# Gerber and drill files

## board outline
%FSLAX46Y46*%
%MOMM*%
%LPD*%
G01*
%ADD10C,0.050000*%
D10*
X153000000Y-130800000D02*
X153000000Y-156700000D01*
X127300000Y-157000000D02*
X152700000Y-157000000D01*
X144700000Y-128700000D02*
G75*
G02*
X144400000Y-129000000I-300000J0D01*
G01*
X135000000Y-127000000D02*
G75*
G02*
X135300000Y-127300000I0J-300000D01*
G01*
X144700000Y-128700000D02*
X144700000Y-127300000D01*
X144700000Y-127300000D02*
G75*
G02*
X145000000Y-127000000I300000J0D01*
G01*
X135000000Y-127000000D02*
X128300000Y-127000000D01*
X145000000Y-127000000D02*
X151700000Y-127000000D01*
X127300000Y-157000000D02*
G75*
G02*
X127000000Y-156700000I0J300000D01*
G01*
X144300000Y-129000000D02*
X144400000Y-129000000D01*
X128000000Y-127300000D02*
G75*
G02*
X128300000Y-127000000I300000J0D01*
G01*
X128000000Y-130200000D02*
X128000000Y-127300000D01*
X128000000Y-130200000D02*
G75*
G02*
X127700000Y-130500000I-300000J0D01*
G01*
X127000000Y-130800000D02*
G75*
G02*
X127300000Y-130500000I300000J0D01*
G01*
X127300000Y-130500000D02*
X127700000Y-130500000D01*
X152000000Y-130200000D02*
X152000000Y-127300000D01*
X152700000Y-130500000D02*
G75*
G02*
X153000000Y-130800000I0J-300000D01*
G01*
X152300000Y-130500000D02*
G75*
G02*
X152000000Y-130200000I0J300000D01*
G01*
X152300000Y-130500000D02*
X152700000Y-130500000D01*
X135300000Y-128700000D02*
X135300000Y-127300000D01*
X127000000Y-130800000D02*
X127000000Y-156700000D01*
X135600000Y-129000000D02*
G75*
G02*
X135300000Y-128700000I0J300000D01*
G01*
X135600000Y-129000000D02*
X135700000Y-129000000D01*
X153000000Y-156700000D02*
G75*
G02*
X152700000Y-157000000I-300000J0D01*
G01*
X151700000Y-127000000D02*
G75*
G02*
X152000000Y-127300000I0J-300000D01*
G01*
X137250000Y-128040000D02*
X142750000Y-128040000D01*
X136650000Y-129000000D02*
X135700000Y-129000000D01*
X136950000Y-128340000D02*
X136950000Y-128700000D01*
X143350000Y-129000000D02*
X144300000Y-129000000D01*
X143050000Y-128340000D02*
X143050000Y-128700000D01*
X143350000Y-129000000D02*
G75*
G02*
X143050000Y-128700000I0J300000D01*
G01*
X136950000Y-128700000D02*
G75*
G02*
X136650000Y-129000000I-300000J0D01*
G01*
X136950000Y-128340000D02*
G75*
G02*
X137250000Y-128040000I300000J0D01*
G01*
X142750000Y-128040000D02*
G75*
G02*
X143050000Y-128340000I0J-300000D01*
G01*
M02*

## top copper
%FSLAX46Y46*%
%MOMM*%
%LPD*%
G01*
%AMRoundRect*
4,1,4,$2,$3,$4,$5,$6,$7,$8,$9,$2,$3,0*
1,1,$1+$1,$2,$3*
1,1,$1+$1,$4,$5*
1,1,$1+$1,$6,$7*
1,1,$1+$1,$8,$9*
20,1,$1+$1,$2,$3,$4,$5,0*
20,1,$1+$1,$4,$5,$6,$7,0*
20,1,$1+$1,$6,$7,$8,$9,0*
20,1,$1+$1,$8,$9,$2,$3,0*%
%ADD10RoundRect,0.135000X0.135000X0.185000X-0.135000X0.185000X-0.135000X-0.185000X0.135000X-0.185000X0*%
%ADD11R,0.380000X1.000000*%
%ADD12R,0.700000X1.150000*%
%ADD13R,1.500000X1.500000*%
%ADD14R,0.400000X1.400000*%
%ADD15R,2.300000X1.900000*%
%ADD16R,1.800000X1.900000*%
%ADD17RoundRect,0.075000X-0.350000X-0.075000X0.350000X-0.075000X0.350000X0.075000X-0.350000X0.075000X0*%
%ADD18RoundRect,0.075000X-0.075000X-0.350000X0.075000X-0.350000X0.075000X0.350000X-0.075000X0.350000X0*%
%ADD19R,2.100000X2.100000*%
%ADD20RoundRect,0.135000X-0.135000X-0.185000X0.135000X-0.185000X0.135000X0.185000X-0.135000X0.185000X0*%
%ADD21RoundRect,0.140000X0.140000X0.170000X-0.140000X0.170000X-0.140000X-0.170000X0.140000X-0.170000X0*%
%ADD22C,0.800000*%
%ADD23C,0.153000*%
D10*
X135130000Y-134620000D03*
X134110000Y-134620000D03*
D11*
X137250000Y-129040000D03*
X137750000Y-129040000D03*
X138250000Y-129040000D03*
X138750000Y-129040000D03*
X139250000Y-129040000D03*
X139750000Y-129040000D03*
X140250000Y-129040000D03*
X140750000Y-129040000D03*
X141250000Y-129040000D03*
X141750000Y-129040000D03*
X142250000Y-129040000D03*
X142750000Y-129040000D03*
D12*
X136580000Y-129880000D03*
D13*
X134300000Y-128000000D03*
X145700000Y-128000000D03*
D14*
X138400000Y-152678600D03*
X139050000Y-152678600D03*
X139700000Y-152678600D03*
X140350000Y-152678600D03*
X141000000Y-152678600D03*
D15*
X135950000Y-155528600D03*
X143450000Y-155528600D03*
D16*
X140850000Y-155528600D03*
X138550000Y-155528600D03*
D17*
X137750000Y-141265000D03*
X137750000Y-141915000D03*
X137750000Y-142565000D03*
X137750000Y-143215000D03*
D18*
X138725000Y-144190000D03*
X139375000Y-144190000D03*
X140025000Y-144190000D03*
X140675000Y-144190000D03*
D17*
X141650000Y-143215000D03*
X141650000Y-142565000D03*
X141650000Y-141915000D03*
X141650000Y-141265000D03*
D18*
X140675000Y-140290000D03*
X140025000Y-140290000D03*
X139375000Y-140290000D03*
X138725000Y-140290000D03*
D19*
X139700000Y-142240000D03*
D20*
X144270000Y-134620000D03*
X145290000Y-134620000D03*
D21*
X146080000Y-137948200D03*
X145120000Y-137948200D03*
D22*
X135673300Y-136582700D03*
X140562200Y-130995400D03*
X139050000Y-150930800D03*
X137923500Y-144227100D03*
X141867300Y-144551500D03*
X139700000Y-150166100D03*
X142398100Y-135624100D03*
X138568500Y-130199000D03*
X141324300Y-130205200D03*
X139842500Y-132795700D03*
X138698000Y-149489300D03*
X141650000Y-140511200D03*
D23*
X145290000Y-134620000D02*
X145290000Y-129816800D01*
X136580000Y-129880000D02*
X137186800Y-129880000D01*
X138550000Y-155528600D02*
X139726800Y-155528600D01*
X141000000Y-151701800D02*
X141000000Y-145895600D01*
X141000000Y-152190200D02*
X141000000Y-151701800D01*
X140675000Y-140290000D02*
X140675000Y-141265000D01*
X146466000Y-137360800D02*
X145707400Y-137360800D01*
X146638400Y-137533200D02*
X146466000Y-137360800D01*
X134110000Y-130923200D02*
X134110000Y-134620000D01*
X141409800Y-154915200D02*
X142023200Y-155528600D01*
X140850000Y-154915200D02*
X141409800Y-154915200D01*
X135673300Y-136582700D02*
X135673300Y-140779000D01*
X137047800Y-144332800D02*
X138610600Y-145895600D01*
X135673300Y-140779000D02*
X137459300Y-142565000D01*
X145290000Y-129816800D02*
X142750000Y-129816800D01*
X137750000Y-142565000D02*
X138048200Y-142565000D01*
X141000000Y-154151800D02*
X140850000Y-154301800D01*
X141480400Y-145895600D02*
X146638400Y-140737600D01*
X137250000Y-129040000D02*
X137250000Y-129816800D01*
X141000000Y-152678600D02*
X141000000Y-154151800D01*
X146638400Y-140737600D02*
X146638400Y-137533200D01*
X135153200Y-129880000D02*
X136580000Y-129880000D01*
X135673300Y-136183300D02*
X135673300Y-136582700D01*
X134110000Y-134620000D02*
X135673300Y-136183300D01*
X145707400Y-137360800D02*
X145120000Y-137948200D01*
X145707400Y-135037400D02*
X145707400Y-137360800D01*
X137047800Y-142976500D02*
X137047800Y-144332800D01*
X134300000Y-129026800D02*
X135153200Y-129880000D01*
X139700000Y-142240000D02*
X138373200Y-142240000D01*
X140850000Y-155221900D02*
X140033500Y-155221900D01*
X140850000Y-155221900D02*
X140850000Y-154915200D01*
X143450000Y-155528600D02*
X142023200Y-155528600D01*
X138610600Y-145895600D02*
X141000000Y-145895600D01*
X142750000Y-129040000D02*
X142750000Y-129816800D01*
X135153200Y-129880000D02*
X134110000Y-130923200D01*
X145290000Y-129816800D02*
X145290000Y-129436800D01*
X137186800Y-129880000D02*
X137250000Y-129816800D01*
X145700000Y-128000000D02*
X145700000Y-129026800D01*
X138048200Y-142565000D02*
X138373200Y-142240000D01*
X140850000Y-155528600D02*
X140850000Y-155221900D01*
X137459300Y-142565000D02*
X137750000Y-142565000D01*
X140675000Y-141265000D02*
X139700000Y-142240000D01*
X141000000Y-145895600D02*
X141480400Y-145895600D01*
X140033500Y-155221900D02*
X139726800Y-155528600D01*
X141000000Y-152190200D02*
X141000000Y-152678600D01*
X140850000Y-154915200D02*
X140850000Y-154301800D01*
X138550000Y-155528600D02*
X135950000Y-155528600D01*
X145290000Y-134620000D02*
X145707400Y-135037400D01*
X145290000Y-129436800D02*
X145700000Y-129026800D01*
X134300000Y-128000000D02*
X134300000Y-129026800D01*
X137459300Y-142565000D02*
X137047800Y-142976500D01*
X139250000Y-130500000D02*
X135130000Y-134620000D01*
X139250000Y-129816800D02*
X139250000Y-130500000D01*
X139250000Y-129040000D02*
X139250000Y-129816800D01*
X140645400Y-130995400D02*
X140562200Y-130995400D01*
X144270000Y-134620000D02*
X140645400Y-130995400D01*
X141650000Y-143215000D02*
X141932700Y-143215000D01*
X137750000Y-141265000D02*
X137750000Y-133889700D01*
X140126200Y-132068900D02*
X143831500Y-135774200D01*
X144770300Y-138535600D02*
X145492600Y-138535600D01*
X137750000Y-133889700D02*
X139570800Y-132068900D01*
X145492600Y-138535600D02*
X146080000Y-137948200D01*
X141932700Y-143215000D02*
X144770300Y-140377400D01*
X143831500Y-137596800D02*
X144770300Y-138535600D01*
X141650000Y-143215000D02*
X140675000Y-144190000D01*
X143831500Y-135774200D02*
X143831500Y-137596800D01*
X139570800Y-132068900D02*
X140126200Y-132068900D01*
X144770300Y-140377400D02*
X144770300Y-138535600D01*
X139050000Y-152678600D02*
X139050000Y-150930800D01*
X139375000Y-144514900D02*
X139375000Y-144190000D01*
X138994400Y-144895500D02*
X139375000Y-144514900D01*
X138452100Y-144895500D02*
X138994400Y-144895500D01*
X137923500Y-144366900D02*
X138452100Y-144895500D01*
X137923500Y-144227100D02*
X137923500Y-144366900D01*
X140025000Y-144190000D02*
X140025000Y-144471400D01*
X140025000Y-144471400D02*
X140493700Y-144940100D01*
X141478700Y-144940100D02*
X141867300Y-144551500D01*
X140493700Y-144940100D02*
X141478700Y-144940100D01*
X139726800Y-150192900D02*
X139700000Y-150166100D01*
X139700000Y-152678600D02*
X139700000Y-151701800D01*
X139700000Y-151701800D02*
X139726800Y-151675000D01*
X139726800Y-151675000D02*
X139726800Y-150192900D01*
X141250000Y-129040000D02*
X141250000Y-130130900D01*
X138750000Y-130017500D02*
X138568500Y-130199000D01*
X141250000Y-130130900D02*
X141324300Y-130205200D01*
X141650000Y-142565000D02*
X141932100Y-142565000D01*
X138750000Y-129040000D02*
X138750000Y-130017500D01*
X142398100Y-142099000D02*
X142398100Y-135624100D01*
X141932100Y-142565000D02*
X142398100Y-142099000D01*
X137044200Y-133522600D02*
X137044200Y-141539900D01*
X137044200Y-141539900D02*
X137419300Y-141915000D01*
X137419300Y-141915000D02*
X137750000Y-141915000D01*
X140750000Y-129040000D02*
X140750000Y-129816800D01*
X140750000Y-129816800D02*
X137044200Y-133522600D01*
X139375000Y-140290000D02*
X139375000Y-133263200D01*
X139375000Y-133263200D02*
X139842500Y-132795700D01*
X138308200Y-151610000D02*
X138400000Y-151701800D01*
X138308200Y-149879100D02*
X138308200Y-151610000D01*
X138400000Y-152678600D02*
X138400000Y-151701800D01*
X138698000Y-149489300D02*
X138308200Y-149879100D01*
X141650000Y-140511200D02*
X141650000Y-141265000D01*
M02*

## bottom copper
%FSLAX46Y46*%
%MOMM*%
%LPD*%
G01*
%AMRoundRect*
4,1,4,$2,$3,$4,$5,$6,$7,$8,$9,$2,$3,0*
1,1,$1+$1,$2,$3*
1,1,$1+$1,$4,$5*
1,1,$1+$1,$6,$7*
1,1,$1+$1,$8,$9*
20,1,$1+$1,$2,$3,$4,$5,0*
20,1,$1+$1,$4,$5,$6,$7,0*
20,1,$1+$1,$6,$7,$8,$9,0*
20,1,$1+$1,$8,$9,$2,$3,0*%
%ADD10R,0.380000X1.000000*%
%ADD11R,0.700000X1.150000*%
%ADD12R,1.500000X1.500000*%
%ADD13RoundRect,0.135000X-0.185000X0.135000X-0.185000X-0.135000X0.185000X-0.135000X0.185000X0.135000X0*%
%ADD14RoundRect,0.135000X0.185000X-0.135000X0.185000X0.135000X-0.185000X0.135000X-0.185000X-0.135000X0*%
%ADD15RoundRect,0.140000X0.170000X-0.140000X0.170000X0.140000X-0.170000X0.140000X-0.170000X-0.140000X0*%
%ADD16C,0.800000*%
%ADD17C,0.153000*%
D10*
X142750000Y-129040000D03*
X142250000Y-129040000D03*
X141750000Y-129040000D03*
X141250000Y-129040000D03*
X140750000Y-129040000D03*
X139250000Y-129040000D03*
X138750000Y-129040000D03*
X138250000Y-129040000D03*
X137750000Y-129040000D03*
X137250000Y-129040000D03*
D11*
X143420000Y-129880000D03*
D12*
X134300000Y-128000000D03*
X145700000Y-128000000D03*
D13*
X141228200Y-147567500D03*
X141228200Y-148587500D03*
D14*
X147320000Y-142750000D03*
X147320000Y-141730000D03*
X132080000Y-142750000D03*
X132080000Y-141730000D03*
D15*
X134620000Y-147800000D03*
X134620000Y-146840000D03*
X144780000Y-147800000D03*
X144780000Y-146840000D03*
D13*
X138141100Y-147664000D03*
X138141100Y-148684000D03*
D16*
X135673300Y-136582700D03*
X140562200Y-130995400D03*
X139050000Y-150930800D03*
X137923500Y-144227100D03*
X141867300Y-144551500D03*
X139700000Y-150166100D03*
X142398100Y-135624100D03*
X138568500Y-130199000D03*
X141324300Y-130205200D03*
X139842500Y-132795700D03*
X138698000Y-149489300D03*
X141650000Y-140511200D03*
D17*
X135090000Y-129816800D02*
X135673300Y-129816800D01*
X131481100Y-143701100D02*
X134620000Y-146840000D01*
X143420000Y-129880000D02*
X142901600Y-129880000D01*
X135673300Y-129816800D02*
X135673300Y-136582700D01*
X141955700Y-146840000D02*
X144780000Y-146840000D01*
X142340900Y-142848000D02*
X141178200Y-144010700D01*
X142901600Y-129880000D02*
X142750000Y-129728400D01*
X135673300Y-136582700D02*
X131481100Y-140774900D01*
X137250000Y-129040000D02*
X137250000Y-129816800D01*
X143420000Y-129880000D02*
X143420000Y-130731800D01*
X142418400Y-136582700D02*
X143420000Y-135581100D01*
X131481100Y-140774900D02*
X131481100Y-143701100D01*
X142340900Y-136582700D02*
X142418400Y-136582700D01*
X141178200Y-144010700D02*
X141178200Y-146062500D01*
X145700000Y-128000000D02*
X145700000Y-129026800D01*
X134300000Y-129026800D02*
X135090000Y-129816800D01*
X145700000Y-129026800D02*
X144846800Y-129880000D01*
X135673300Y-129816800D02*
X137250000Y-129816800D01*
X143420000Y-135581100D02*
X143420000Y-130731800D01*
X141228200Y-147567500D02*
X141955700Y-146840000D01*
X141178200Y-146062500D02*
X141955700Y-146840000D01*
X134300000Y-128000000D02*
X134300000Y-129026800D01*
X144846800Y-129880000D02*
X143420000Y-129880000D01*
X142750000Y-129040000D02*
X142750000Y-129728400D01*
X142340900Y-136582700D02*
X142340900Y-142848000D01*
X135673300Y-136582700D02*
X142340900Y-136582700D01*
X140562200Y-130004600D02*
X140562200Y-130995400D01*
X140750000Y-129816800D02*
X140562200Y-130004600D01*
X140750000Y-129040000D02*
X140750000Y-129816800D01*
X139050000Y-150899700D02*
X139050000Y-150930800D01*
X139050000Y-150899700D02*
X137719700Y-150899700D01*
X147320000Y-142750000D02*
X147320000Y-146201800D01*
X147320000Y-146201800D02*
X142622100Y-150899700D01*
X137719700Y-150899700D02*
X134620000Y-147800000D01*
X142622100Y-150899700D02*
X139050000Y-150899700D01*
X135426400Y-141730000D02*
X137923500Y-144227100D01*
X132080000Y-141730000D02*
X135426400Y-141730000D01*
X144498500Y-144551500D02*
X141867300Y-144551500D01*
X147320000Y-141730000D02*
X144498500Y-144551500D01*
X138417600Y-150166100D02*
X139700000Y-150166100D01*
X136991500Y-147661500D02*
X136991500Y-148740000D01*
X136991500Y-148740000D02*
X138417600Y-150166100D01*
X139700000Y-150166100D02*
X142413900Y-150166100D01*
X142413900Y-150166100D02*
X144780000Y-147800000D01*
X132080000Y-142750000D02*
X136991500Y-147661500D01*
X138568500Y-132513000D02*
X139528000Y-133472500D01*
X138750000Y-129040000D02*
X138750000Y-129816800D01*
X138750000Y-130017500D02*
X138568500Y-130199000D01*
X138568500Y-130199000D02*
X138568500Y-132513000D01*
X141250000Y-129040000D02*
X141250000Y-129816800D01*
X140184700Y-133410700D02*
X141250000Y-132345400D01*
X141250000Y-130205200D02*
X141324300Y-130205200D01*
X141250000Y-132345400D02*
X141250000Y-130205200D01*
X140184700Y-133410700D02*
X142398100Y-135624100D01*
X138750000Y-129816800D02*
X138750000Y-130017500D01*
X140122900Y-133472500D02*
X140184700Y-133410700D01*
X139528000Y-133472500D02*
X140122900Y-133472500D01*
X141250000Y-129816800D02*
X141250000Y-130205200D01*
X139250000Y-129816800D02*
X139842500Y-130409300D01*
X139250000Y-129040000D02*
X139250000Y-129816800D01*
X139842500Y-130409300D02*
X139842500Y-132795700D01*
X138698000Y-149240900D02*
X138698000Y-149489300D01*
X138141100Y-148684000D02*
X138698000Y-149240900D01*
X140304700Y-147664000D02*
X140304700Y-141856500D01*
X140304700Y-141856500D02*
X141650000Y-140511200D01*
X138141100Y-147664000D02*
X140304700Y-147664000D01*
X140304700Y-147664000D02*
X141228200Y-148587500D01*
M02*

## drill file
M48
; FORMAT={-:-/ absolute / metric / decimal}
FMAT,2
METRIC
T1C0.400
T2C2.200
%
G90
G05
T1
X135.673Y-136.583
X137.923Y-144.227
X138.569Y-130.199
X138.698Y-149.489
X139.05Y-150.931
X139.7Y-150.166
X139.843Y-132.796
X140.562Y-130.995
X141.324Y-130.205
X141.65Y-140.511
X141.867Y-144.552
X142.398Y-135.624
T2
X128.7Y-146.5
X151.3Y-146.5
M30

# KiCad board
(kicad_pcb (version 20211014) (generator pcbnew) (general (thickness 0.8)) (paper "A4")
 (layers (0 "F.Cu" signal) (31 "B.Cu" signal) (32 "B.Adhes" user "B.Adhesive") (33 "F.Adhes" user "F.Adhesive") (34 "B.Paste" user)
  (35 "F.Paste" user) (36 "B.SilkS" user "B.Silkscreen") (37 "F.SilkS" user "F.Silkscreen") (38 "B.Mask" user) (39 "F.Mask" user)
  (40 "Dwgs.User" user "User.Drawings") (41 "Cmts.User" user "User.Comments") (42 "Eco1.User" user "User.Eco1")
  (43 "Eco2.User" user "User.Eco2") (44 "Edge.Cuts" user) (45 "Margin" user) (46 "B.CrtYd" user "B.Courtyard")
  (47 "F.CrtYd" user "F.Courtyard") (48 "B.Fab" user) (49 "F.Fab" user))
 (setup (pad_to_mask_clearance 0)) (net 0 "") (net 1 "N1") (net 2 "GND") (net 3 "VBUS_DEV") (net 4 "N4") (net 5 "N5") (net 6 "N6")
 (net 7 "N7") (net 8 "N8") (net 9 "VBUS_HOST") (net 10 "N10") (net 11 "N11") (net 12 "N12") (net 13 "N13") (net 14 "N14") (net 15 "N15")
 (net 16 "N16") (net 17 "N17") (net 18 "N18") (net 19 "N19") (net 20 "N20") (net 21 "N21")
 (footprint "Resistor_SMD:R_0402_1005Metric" (layer "F.Cu") (at 134.62 134.62 180)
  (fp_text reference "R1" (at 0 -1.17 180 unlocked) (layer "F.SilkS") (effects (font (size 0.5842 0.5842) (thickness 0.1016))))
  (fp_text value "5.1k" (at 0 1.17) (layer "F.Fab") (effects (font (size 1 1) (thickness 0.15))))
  (pad "1" smd roundrect (at -0.51 0 180) (size 0.54 0.64) (layers "F.Cu" "F.Paste" "F.Mask") (roundrect_rratio 0.25) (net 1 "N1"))
  (pad "2" smd roundrect (at 0.51 0 180) (size 0.54 0.64) (layers "F.Cu" "F.Paste" "F.Mask") (roundrect_rratio 0.25) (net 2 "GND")))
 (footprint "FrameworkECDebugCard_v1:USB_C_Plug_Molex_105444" (layer "F.Cu") (at 140 129)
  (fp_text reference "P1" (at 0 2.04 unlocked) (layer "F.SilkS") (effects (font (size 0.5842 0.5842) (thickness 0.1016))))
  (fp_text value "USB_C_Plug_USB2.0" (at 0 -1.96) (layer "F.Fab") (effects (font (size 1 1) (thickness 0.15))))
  (fp_line (start -2.75 -0.96) (end 2.75 -0.96) (layer "Edge.Cuts") (width 0.05))
  (fp_line (start -3.35 0) (end -4.3 0) (layer "Edge.Cuts") (width 0.05))
  (fp_line (start -3.05 -0.66) (end -3.05 -0.3) (layer "Edge.Cuts") (width 0.05))
  (fp_line (start 3.35 0) (end 4.3 0) (layer "Edge.Cuts") (width 0.05))
  (fp_line (start 3.05 -0.66) (end 3.05 -0.3) (layer "Edge.Cuts") (width 0.05))
  (fp_arc (start 3.35 0) (mid 3.137868 -0.087868) (end 3.05 -0.3) (layer "Edge.Cuts") (width 0.05))
  (fp_arc (start -3.05 -0.3) (mid -3.137868 -0.087868) (end -3.35 0) (layer "Edge.Cuts") (width 0.05))
  (fp_arc (start -3.05 -0.66) (mid -2.962132 -0.872132) (end -2.75 -0.96) (layer "Edge.Cuts") (width 0.05))
  (fp_arc (start 2.75 -0.96) (mid 2.962132 -0.872132) (end 3.05 -0.66) (layer "Edge.Cuts") (width 0.05))
  (pad "A1" smd rect locked (at -2.75 0.04) (size 0.38 1) (layers "F.Cu" "F.Paste" "F.Mask") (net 2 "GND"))
  (pad "A2" smd rect locked (at -2.25 0.04) (size 0.38 1) (layers "F.Cu" "F.Paste" "F.Mask"))
  (pad "A3" smd rect locked (at -1.75 0.04) (size 0.38 1) (layers "F.Cu" "F.Paste" "F.Mask"))
  (pad "A4" smd rect locked (at -1.25 0.04) (size 0.38 1) (layers "F.Cu" "F.Paste" "F.Mask") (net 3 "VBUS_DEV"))
  (pad "A5" smd rect locked (at -0.75 0.04) (size 0.38 1) (layers "F.Cu" "F.Paste" "F.Mask") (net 1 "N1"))
  (pad "A6" smd rect locked (at -0.25 0.04) (size 0.38 1) (layers "F.Cu" "F.Paste" "F.Mask") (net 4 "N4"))
  (pad "A7" smd rect locked (at 0.25 0.04) (size 0.38 1) (layers "F.Cu" "F.Paste" "F.Mask") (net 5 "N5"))
  (pad "A8" smd rect locked (at 0.75 0.04) (size 0.38 1) (layers "F.Cu" "F.Paste" "F.Mask") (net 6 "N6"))
  (pad "A9" smd rect locked (at 1.25 0.04) (size 0.38 1) (layers "F.Cu" "F.Paste" "F.Mask") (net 3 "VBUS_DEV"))
  (pad "A10" smd rect locked (at 1.75 0.04) (size 0.38 1) (layers "F.Cu" "F.Paste" "F.Mask"))
  (pad "A11" smd rect locked (at 2.25 0.04) (size 0.38 1) (layers "F.Cu" "F.Paste" "F.Mask"))
  (pad "A12" smd rect locked (at 2.75 0.04) (size 0.38 1) (layers "F.Cu" "F.Paste" "F.Mask") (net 2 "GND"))
  (pad "B1" smd rect locked (at 2.75 0.04) (size 0.38 1) (layers "B.Cu" "B.Paste" "B.Mask") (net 2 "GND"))
  (pad "B2" smd rect locked (at 2.25 0.04) (size 0.38 1) (layers "B.Cu" "B.Paste" "B.Mask"))
  (pad "B3" smd rect locked (at 1.75 0.04) (size 0.38 1) (layers "B.Cu" "B.Paste" "B.Mask"))
  (pad "B4" smd rect locked (at 1.25 0.04) (size 0.38 1) (layers "B.Cu" "B.Paste" "B.Mask") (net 3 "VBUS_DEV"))
  (pad "B5" smd rect locked (at 0.75 0.04) (size 0.38 1) (layers "B.Cu" "B.Paste" "B.Mask") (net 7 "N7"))
  (pad "B8" smd rect locked (at -0.75 0.04) (size 0.38 1) (layers "B.Cu" "B.Paste" "B.Mask") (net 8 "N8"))
  (pad "B9" smd rect locked (at -1.25 0.04) (size 0.38 1) (layers "B.Cu" "B.Paste" "B.Mask") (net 3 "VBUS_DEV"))
  (pad "B10" smd rect locked (at -1.75 0.04) (size 0.38 1) (layers "B.Cu" "B.Paste" "B.Mask"))
  (pad "B11" smd rect locked (at -2.25 0.04) (size 0.38 1) (layers "B.Cu" "B.Paste" "B.Mask"))
  (pad "B12" smd rect locked (at -2.75 0.04) (size 0.38 1) (layers "B.Cu" "B.Paste" "B.Mask") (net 2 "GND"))
  (pad "S1" smd rect locked (at 3.42 0.88) (size 0.7 1.15) (layers "B.Cu" "B.Paste" "B.Mask") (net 2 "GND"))
  (pad "S1" smd rect locked (at -3.42 0.88) (size 0.7 1.15) (layers "F.Cu" "F.Paste" "F.Mask") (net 2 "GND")))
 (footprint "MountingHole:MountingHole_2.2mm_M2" (layer "F.Cu") (at 128.7 146.5)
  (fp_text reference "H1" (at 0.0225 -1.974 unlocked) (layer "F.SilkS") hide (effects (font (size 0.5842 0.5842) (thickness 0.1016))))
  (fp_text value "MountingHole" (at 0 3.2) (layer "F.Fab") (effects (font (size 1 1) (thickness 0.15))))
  (pad "" np_thru_hole circle locked (at 0 0) (size 2.2 2.2) (drill 2.2) (layers *.Cu *.Mask)))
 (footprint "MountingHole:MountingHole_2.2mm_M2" (layer "F.Cu") (at 151.3 146.5)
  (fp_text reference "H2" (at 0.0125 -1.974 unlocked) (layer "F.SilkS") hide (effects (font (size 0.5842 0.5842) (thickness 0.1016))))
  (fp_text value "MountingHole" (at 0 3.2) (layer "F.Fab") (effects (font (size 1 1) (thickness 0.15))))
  (pad "" np_thru_hole circle locked (at 0 0) (size 2.2 2.2) (drill 2.2) (layers *.Cu *.Mask)))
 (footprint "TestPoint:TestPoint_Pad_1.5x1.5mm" (layer "F.Cu") (at 134.3 128)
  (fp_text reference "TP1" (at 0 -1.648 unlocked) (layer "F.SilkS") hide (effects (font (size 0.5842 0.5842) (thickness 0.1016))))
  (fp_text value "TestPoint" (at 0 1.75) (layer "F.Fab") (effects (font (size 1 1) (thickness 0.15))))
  (pad "1" smd rect locked (at 0 0) (size 1.5 1.5) (layers "F.Cu" "F.Mask") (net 2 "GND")))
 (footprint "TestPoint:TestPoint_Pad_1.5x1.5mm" (layer "F.Cu") (at 145.7 128)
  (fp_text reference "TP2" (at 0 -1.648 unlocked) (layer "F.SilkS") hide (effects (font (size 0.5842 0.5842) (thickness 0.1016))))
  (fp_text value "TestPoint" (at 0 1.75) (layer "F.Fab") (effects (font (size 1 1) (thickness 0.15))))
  (pad "1" smd rect locked (at 0 0) (size 1.5 1.5) (layers "F.Cu" "F.Mask") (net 2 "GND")))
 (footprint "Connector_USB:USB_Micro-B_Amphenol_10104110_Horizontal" (layer "F.Cu") (at 139.7 154.2286)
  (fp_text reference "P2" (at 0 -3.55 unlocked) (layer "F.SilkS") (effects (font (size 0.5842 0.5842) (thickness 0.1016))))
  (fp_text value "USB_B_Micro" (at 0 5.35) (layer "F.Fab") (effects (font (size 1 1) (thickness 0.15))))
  (pad "1" smd rect (at -1.3 -1.55) (size 0.4 1.4) (layers "F.Cu" "F.Paste" "F.Mask") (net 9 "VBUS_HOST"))
  (pad "2" smd rect (at -0.65 -1.55) (size 0.4 1.4) (layers "F.Cu" "F.Paste" "F.Mask") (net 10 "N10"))
  (pad "3" smd rect (at 0 -1.55) (size 0.4 1.4) (layers "F.Cu" "F.Paste" "F.Mask") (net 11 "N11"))
  (pad "4" smd rect (at 0.65 -1.55) (size 0.4 1.4) (layers "F.Cu" "F.Paste" "F.Mask") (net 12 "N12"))
  (pad "5" smd rect (at 1.3 -1.55) (size 0.4 1.4) (layers "F.Cu" "F.Paste" "F.Mask") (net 2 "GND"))
  (pad "6" smd rect (at -3.75 1.3) (size 2.3 1.9) (layers "F.Cu" "F.Paste" "F.Mask") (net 2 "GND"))
  (pad "6" smd rect (at 3.75 1.3) (size 2.3 1.9) (layers "F.Cu" "F.Paste" "F.Mask") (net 2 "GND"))
  (pad "6" smd rect (at 1.15 1.3) (size 1.8 1.9) (layers "F.Cu" "F.Paste" "F.Mask") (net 2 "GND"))
  (pad "6" smd rect (at -1.15 1.3) (size 1.8 1.9) (layers "F.Cu" "F.Paste" "F.Mask") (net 2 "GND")))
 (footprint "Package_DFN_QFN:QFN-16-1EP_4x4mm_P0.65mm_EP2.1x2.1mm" (layer "F.Cu") (at 139.7 142.24)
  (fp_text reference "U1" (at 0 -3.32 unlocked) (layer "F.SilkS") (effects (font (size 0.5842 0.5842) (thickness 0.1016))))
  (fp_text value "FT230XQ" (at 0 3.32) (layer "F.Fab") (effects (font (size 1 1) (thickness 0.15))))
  (pad "" smd roundrect (at -0.525 0.525) (size 0.85 0.85) (layers "F.Paste") (roundrect_rratio 0.25))
  (pad "" smd roundrect (at 0.525 -0.525) (size 0.85 0.85) (layers "F.Paste") (roundrect_rratio 0.25))
  (pad "" smd roundrect (at -0.525 -0.525) (size 0.85 0.85) (layers "F.Paste") (roundrect_rratio 0.25))
  (pad "" smd roundrect (at 0.525 0.525) (size 0.85 0.85) (layers "F.Paste") (roundrect_rratio 0.25))
  (pad "1" smd roundrect (at -1.95 -0.975) (size 0.85 0.3) (layers "F.Cu" "F.Paste" "F.Mask") (roundrect_rratio 0.25) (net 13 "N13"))
  (pad "2" smd roundrect (at -1.95 -0.325) (size 0.85 0.3) (layers "F.Cu" "F.Paste" "F.Mask") (roundrect_rratio 0.25) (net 6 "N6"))
  (pad "3" smd roundrect (at -1.95 0.325) (size 0.85 0.3) (layers "F.Cu" "F.Paste" "F.Mask") (roundrect_rratio 0.25) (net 2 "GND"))
  (pad "4" smd roundrect (at -1.95 0.975) (size 0.85 0.3) (layers "F.Cu" "F.Paste" "F.Mask") (roundrect_rratio 0.25) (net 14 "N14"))
  (pad "5" smd roundrect (at -0.975 1.95) (size 0.3 0.85) (layers "F.Cu" "F.Paste" "F.Mask") (roundrect_rratio 0.25) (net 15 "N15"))
  (pad "6" smd roundrect (at -0.325 1.95) (size 0.3 0.85) (layers "F.Cu" "F.Paste" "F.Mask") (roundrect_rratio 0.25) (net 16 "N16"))
  (pad "7" smd roundrect (at 0.325 1.95) (size 0.3 0.85) (layers "F.Cu" "F.Paste" "F.Mask") (roundrect_rratio 0.25) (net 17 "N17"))
  (pad "8" smd roundrect (at 0.975 1.95) (size 0.3 0.85) (layers "F.Cu" "F.Paste" "F.Mask") (roundrect_rratio 0.25) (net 13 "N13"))
  (pad "9" smd roundrect (at 1.95 0.975) (size 0.85 0.3) (layers "F.Cu" "F.Paste" "F.Mask") (roundrect_rratio 0.25) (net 13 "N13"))
  (pad "10" smd roundrect (at 1.95 0.325) (size 0.85 0.3) (layers "F.Cu" "F.Paste" "F.Mask") (roundrect_rratio 0.25) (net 3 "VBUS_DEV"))
  (pad "11" smd roundrect (at 1.95 -0.325) (size 0.85 0.3) (layers "F.Cu" "F.Paste" "F.Mask") (roundrect_rratio 0.25) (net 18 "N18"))
  (pad "12" smd roundrect (at 1.95 -0.975) (size 0.85 0.3) (layers "F.Cu" "F.Paste" "F.Mask") (roundrect_rratio 0.25) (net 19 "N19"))
  (pad "13" smd roundrect (at 0.975 -1.95) (size 0.3 0.85) (layers "F.Cu" "F.Paste" "F.Mask") (roundrect_rratio 0.25) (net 2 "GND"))
  (pad "14" smd roundrect (at 0.325 -1.95) (size 0.3 0.85) (layers "F.Cu" "F.Paste" "F.Mask") (roundrect_rratio 0.25) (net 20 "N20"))
  (pad "15" smd roundrect (at -0.325 -1.95) (size 0.3 0.85) (layers "F.Cu" "F.Paste" "F.Mask") (roundrect_rratio 0.25) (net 8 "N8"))
  (pad "16" smd roundrect (at -0.975 -1.95) (size 0.3 0.85) (layers "F.Cu" "F.Paste" "F.Mask") (roundrect_rratio 0.25) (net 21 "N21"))
  (pad "17" smd rect (at 0 0) (size 2.1 2.1) (layers "F.Cu" "F.Mask") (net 2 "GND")))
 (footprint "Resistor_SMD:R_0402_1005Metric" (layer "F.Cu") (at 144.78 134.62)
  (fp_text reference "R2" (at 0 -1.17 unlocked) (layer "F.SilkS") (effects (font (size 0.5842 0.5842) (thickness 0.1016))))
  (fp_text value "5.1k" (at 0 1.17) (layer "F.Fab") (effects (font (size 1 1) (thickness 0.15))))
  (pad "1" smd roundrect (at -0.51 0) (size 0.54 0.64) (layers "F.Cu" "F.Paste" "F.Mask") (roundrect_rratio 0.25) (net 7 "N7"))
  (pad "2" smd roundrect (at 0.51 0) (size 0.54 0.64) (layers "F.Cu" "F.Paste" "F.Mask") (roundrect_rratio 0.25) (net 2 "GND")))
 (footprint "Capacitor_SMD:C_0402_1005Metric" (layer "F.Cu") (at 145.6 137.9482 180)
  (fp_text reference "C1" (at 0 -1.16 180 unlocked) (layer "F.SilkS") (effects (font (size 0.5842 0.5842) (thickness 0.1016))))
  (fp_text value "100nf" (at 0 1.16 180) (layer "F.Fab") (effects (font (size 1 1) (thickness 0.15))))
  (pad "1" smd roundrect (at -0.48 0 180) (size 0.56 0.62) (layers "F.Cu" "F.Paste" "F.Mask") (roundrect_rratio 0.25) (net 13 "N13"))
  (pad "2" smd roundrect (at 0.48 0 180) (size 0.56 0.62) (layers "F.Cu" "F.Paste" "F.Mask") (roundrect_rratio 0.25) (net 2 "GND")))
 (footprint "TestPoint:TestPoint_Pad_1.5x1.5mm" (layer "B.Cu") (at 134.3 128)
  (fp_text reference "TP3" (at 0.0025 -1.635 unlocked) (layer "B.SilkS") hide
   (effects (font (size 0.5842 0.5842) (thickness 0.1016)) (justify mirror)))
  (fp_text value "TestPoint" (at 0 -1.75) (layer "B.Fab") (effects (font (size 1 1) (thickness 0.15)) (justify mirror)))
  (pad "1" smd rect locked (at 0 0) (size 1.5 1.5) (layers "B.Cu" "B.Mask") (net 2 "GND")))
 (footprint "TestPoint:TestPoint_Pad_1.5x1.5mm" (layer "B.Cu") (at 145.7 128)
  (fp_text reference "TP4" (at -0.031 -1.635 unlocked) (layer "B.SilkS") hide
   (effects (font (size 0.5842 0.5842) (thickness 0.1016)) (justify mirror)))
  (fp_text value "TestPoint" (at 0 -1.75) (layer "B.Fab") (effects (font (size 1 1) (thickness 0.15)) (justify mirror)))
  (pad "1" smd rect locked (at 0 0) (size 1.5 1.5) (layers "B.Cu" "B.Mask") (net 2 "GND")))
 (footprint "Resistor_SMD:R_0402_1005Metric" (layer "B.Cu") (at 141.2282 148.0775 -90)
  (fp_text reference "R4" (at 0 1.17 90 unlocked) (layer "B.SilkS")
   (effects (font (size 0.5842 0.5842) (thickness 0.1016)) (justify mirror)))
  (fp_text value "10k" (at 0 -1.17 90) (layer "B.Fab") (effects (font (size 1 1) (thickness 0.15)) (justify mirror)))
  (pad "1" smd roundrect (at -0.51 0 270) (size 0.54 0.64) (layers "B.Cu" "B.Paste" "B.Mask") (roundrect_rratio 0.25) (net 2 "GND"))
  (pad "2" smd roundrect (at 0.51 0 270) (size 0.54 0.64) (layers "B.Cu" "B.Paste" "B.Mask") (roundrect_rratio 0.25) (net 19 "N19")))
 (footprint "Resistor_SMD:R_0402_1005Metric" (layer "B.Cu") (at 147.32 142.24 90)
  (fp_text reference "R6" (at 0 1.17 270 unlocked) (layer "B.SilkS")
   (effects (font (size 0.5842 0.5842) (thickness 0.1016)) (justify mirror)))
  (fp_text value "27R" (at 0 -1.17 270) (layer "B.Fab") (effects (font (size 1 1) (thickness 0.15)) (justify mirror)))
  (pad "1" smd roundrect (at -0.51 0 90) (size 0.54 0.64) (layers "B.Cu" "B.Paste" "B.Mask") (roundrect_rratio 0.25) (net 10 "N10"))
  (pad "2" smd roundrect (at 0.51 0 90) (size 0.54 0.64) (layers "B.Cu" "B.Paste" "B.Mask") (roundrect_rratio 0.25) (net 17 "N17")))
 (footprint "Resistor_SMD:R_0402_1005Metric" (layer "B.Cu") (at 132.08 142.24 90)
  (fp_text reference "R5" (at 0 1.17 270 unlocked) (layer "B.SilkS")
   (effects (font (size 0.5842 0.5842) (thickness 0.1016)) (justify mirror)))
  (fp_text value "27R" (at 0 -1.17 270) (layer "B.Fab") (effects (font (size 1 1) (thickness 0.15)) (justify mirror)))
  (pad "1" smd roundrect (at -0.51 0 90) (size 0.54 0.64) (layers "B.Cu" "B.Paste" "B.Mask") (roundrect_rratio 0.25) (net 11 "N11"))
  (pad "2" smd roundrect (at 0.51 0 90) (size 0.54 0.64) (layers "B.Cu" "B.Paste" "B.Mask") (roundrect_rratio 0.25) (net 16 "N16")))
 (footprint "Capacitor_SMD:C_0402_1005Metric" (layer "B.Cu") (at 134.62 147.32 90)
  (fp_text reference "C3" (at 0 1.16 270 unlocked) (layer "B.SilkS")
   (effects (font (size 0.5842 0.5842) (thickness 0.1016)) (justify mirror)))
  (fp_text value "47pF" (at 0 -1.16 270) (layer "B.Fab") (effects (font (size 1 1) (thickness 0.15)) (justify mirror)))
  (pad "1" smd roundrect (at -0.48 0 90) (size 0.56 0.62) (layers "B.Cu" "B.Paste" "B.Mask") (roundrect_rratio 0.25) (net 10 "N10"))
  (pad "2" smd roundrect (at 0.48 0 90) (size 0.56 0.62) (layers "B.Cu" "B.Paste" "B.Mask") (roundrect_rratio 0.25) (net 2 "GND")))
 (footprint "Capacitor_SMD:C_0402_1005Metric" (layer "B.Cu") (at 144.78 147.32 90)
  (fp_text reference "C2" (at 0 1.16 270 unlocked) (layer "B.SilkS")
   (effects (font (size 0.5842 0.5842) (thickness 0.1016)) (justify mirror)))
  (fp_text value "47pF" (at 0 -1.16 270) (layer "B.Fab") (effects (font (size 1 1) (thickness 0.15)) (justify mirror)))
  (pad "1" smd roundrect (at -0.48 0 90) (size 0.56 0.62) (layers "B.Cu" "B.Paste" "B.Mask") (roundrect_rratio 0.25) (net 11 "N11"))
  (pad "2" smd roundrect (at 0.48 0 90) (size 0.56 0.62) (layers "B.Cu" "B.Paste" "B.Mask") (roundrect_rratio 0.25) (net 2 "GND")))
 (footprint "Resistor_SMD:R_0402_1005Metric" (layer "B.Cu") (at 138.1411 148.174 -90)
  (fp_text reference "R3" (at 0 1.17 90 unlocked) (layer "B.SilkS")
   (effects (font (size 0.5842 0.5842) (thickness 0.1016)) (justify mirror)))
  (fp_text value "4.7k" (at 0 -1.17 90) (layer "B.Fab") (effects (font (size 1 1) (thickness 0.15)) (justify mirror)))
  (pad "1" smd roundrect (at -0.51 0 270) (size 0.54 0.64) (layers "B.Cu" "B.Paste" "B.Mask") (roundrect_rratio 0.25) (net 19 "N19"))
  (pad "2" smd roundrect (at 0.51 0 270) (size 0.54 0.64) (layers "B.Cu" "B.Paste" "B.Mask") (roundrect_rratio 0.25) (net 9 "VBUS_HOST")))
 (gr_line (start 153 130.8) (end 153 156.7) (layer "Edge.Cuts") (width 0.05))
 (gr_line (start 127.3 157) (end 152.7 157) (layer "Edge.Cuts") (width 0.05))
 (gr_arc (start 144.7 128.7) (mid 144.612132 128.912132) (end 144.4 129) (layer "Edge.Cuts") (width 0.05))
 (gr_arc (start 135 127) (mid 135.212132 127.087868) (end 135.3 127.3) (layer "Edge.Cuts") (width 0.05))
 (gr_line (start 144.7 128.7) (end 144.7 127.3) (layer "Edge.Cuts") (width 0.05))
 (gr_arc (start 144.7 127.3) (mid 144.787868 127.087868) (end 145 127) (layer "Edge.Cuts") (width 0.05))
 (gr_line (start 135 127) (end 128.3 127) (layer "Edge.Cuts") (width 0.05))
 (gr_line (start 145 127) (end 151.7 127) (layer "Edge.Cuts") (width 0.05))
 (gr_arc (start 127.3 157) (mid 127.087868 156.912132) (end 127 156.7) (layer "Edge.Cuts") (width 0.05))
 (gr_line (start 144.3 129) (end 144.4 129) (layer "Edge.Cuts") (width 0.05))
 (gr_arc (start 128 127.3) (mid 128.087868 127.087868) (end 128.3 127) (layer "Edge.Cuts") (width 0.05))
 (gr_line (start 128 130.2) (end 128 127.3) (layer "Edge.Cuts") (width 0.05))
 (gr_arc (start 128 130.2) (mid 127.912132 130.412132) (end 127.7 130.5) (layer "Edge.Cuts") (width 0.05))
 (gr_arc (start 127 130.8) (mid 127.087868 130.587868) (end 127.3 130.5) (layer "Edge.Cuts") (width 0.05))
 (gr_line (start 127.3 130.5) (end 127.7 130.5) (layer "Edge.Cuts") (width 0.05))
 (gr_line (start 152 130.2) (end 152 127.3) (layer "Edge.Cuts") (width 0.05))
 (gr_arc (start 152.7 130.5) (mid 152.912132 130.587868) (end 153 130.8) (layer "Edge.Cuts") (width 0.05))
 (gr_arc (start 152.3 130.5) (mid 152.087868 130.412132) (end 152 130.2) (layer "Edge.Cuts") (width 0.05))
 (gr_line (start 152.3 130.5) (end 152.7 130.5) (layer "Edge.Cuts") (width 0.05))
 (gr_line (start 135.3 128.7) (end 135.3 127.3) (layer "Edge.Cuts") (width 0.05))
 (gr_line (start 127 130.8) (end 127 156.7) (layer "Edge.Cuts") (width 0.05))
 (gr_arc (start 135.6 129) (mid 135.387868 128.912132) (end 135.3 128.7) (layer "Edge.Cuts") (width 0.05))
 (gr_line (start 135.6 129) (end 135.7 129) (layer "Edge.Cuts") (width 0.05))
 (gr_arc (start 153 156.7) (mid 152.912132 156.912132) (end 152.7 157) (layer "Edge.Cuts") (width 0.05))
 (gr_arc (start 151.7 127) (mid 151.912132 127.087868) (end 152 127.3) (layer "Edge.Cuts") (width 0.05))
 (segment (start 145.29 134.62) (end 145.29 129.8168) (width 0.153) (layer "F.Cu") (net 2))
 (segment (start 136.58 129.88) (end 137.1868 129.88) (width 0.153) (layer "F.Cu") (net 2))
 (segment (start 138.55 155.5286) (end 139.7268 155.5286) (width 0.153) (layer "F.Cu") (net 2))
 (segment (start 141 151.7018) (end 141 145.8956) (width 0.153) (layer "F.Cu") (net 2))
 (segment (start 141 152.1902) (end 141 151.7018) (width 0.153) (layer "F.Cu") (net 2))
 (segment (start 140.675 140.29) (end 140.675 141.265) (width 0.153) (layer "F.Cu") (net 2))
 (segment (start 146.466 137.3608) (end 145.7074 137.3608) (width 0.153) (layer "F.Cu") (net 2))
 (segment (start 146.6384 137.5332) (end 146.466 137.3608) (width 0.153) (layer "F.Cu") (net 2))
 (segment (start 134.11 130.9232) (end 134.11 134.62) (width 0.153) (layer "F.Cu") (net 2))
 (segment (start 141.4098 154.9152) (end 142.0232 155.5286) (width 0.153) (layer "F.Cu") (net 2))
 (segment (start 140.85 154.9152) (end 141.4098 154.9152) (width 0.153) (layer "F.Cu") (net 2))
 (segment (start 135.6733 136.5827) (end 135.6733 140.779) (width 0.153) (layer "F.Cu") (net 2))
 (segment (start 137.0478 144.3328) (end 138.6106 145.8956) (width 0.153) (layer "F.Cu") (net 2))
 (segment (start 135.6733 140.779) (end 137.4593 142.565) (width 0.153) (layer "F.Cu") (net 2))
 (segment (start 145.29 129.8168) (end 142.75 129.8168) (width 0.153) (layer "F.Cu") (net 2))
 (segment (start 137.75 142.565) (end 138.0482 142.565) (width 0.153) (layer "F.Cu") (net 2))
 (segment (start 141 154.1518) (end 140.85 154.3018) (width 0.153) (layer "F.Cu") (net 2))
 (segment (start 141.4804 145.8956) (end 146.6384 140.7376) (width 0.153) (layer "F.Cu") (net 2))
 (segment (start 137.25 129.04) (end 137.25 129.8168) (width 0.153) (layer "F.Cu") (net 2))
 (segment (start 141 152.6786) (end 141 154.1518) (width 0.153) (layer "F.Cu") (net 2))
 (segment (start 146.6384 140.7376) (end 146.6384 137.5332) (width 0.153) (layer "F.Cu") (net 2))
 (segment (start 135.1532 129.88) (end 136.58 129.88) (width 0.153) (layer "F.Cu") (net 2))
 (segment (start 135.6733 136.1833) (end 135.6733 136.5827) (width 0.153) (layer "F.Cu") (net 2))
 (segment (start 134.11 134.62) (end 135.6733 136.1833) (width 0.153) (layer "F.Cu") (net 2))
 (segment (start 145.7074 137.3608) (end 145.12 137.9482) (width 0.153) (layer "F.Cu") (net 2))
 (segment (start 145.7074 135.0374) (end 145.7074 137.3608) (width 0.153) (layer "F.Cu") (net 2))
 (segment (start 137.0478 142.9765) (end 137.0478 144.3328) (width 0.153) (layer "F.Cu") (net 2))
 (segment (start 134.3 129.0268) (end 135.1532 129.88) (width 0.153) (layer "F.Cu") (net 2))
 (segment (start 139.7 142.24) (end 138.3732 142.24) (width 0.153) (layer "F.Cu") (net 2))
 (segment (start 140.85 155.2219) (end 140.0335 155.2219) (width 0.153) (layer "F.Cu") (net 2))
 (segment (start 140.85 155.2219) (end 140.85 154.9152) (width 0.153) (layer "F.Cu") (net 2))
 (segment (start 143.45 155.5286) (end 142.0232 155.5286) (width 0.153) (layer "F.Cu") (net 2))
 (segment (start 138.6106 145.8956) (end 141 145.8956) (width 0.153) (layer "F.Cu") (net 2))
 (segment (start 142.75 129.04) (end 142.75 129.8168) (width 0.153) (layer "F.Cu") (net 2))
 (segment (start 135.1532 129.88) (end 134.11 130.9232) (width 0.153) (layer "F.Cu") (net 2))
 (segment (start 145.29 129.8168) (end 145.29 129.4368) (width 0.153) (layer "F.Cu") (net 2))
 (segment (start 137.1868 129.88) (end 137.25 129.8168) (width 0.153) (layer "F.Cu") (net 2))
 (segment (start 145.7 128) (end 145.7 129.0268) (width 0.153) (layer "F.Cu") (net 2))
 (segment (start 138.0482 142.565) (end 138.3732 142.24) (width 0.153) (layer "F.Cu") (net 2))
 (segment (start 140.85 155.5286) (end 140.85 155.2219) (width 0.153) (layer "F.Cu") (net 2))
 (segment (start 137.4593 142.565) (end 137.75 142.565) (width 0.153) (layer "F.Cu") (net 2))
 (segment (start 140.675 141.265) (end 139.7 142.24) (width 0.153) (layer "F.Cu") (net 2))
 (segment (start 141 145.8956) (end 141.4804 145.8956) (width 0.153) (layer "F.Cu") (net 2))
 (segment (start 140.0335 155.2219) (end 139.7268 155.5286) (width 0.153) (layer "F.Cu") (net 2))
 (segment (start 141 152.1902) (end 141 152.6786) (width 0.153) (layer "F.Cu") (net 2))
 (segment (start 140.85 154.9152) (end 140.85 154.3018) (width 0.153) (layer "F.Cu") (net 2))
 (segment (start 138.55 155.5286) (end 135.95 155.5286) (width 0.153) (layer "F.Cu") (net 2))
 (segment (start 145.29 134.62) (end 145.7074 135.0374) (width 0.153) (layer "F.Cu") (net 2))
 (segment (start 145.29 129.4368) (end 145.7 129.0268) (width 0.153) (layer "F.Cu") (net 2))
 (segment (start 134.3 128) (end 134.3 129.0268) (width 0.153) (layer "F.Cu") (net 2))
 (segment (start 137.4593 142.565) (end 137.0478 142.9765) (width 0.153) (layer "F.Cu") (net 2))
 (via (at 135.6733 136.5827) (size 0.8) (drill 0.4) (layers "F.Cu" "B.Cu") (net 2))
 (segment (start 135.09 129.8168) (end 135.6733 129.8168) (width 0.153) (layer "B.Cu") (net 2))
 (segment (start 131.4811 143.7011) (end 134.62 146.84) (width 0.153) (layer "B.Cu") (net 2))
 (segment (start 143.42 129.88) (end 142.9016 129.88) (width 0.153) (layer "B.Cu") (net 2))
 (segment (start 135.6733 129.8168) (end 135.6733 136.5827) (width 0.153) (layer "B.Cu") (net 2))
 (segment (start 141.9557 146.84) (end 144.78 146.84) (width 0.153) (layer "B.Cu") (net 2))
 (segment (start 142.3409 142.848) (end 141.1782 144.0107) (width 0.153) (layer "B.Cu") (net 2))
 (segment (start 142.9016 129.88) (end 142.75 129.7284) (width 0.153) (layer "B.Cu") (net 2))
 (segment (start 135.6733 136.5827) (end 131.4811 140.7749) (width 0.153) (layer "B.Cu") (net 2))
 (segment (start 137.25 129.04) (end 137.25 129.8168) (width 0.153) (layer "B.Cu") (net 2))
 (segment (start 143.42 129.88) (end 143.42 130.7318) (width 0.153) (layer "B.Cu") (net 2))
 (segment (start 142.4184 136.5827) (end 143.42 135.5811) (width 0.153) (layer "B.Cu") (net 2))
 (segment (start 131.4811 140.7749) (end 131.4811 143.7011) (width 0.153) (layer "B.Cu") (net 2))
 (segment (start 142.3409 136.5827) (end 142.4184 136.5827) (width 0.153) (layer "B.Cu") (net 2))
 (segment (start 141.1782 144.0107) (end 141.1782 146.0625) (width 0.153) (layer "B.Cu") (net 2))
 (segment (start 145.7 128) (end 145.7 129.0268) (width 0.153) (layer "B.Cu") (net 2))
 (segment (start 134.3 129.0268) (end 135.09 129.8168) (width 0.153) (layer "B.Cu") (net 2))
 (segment (start 145.7 129.0268) (end 144.8468 129.88) (width 0.153) (layer "B.Cu") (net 2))
 (segment (start 135.6733 129.8168) (end 137.25 129.8168) (width 0.153) (layer "B.Cu") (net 2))
 (segment (start 143.42 135.5811) (end 143.42 130.7318) (width 0.153) (layer "B.Cu") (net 2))
 (segment (start 141.2282 147.5675) (end 141.9557 146.84) (width 0.153) (layer "B.Cu") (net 2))
 (segment (start 141.1782 146.0625) (end 141.9557 146.84) (width 0.153) (layer "B.Cu") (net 2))
 (segment (start 134.3 128) (end 134.3 129.0268) (width 0.153) (layer "B.Cu") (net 2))
 (segment (start 144.8468 129.88) (end 143.42 129.88) (width 0.153) (layer "B.Cu") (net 2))
 (segment (start 142.75 129.04) (end 142.75 129.7284) (width 0.153) (layer "B.Cu") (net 2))
 (segment (start 142.3409 136.5827) (end 142.3409 142.848) (width 0.153) (layer "B.Cu") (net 2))
 (segment (start 135.6733 136.5827) (end 142.3409 136.5827) (width 0.153) (layer "B.Cu") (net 2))
 (segment (start 139.25 130.5) (end 135.13 134.62) (width 0.153) (layer "F.Cu") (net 1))
 (segment (start 139.25 129.8168) (end 139.25 130.5) (width 0.153) (layer "F.Cu") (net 1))
 (segment (start 139.25 129.04) (end 139.25 129.8168) (width 0.153) (layer "F.Cu") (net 1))
 (segment (start 140.6454 130.9954) (end 140.5622 130.9954) (width 0.153) (layer "F.Cu") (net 7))
 (segment (start 144.27 134.62) (end 140.6454 130.9954) (width 0.153) (layer "F.Cu") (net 7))
 (via (at 140.5622 130.9954) (size 0.8) (drill 0.4) (layers "F.Cu" "B.Cu") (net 7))
 (segment (start 140.5622 130.0046) (end 140.5622 130.9954) (width 0.153) (layer "B.Cu") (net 7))
 (segment (start 140.75 129.8168) (end 140.5622 130.0046) (width 0.153) (layer "B.Cu") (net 7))
 (segment (start 140.75 129.04) (end 140.75 129.8168) (width 0.153) (layer "B.Cu") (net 7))
 (segment (start 141.65 143.215) (end 141.9327 143.215) (width 0.153) (layer "F.Cu") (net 13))
 (segment (start 137.75 141.265) (end 137.75 133.8897) (width 0.153) (layer "F.Cu") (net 13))
 (segment (start 140.1262 132.0689) (end 143.8315 135.7742) (width 0.153) (layer "F.Cu") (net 13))
 (segment (start 144.7703 138.5356) (end 145.4926 138.5356) (width 0.153) (layer "F.Cu") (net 13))
 (segment (start 137.75 133.8897) (end 139.5708 132.0689) (width 0.153) (layer "F.Cu") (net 13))
 (segment (start 145.4926 138.5356) (end 146.08 137.9482) (width 0.153) (layer "F.Cu") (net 13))
 (segment (start 141.9327 143.215) (end 144.7703 140.3774) (width 0.153) (layer "F.Cu") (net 13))
 (segment (start 143.8315 137.5968) (end 144.7703 138.5356) (width 0.153) (layer "F.Cu") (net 13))
 (segment (start 141.65 143.215) (end 140.675 144.19) (width 0.153) (layer "F.Cu") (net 13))
 (segment (start 143.8315 135.7742) (end 143.8315 137.5968) (width 0.153) (layer "F.Cu") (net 13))
 (segment (start 139.5708 132.0689) (end 140.1262 132.0689) (width 0.153) (layer "F.Cu") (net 13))
 (segment (start 144.7703 140.3774) (end 144.7703 138.5356) (width 0.153) (layer "F.Cu") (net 13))
 (segment (start 139.05 152.6786) (end 139.05 150.9308) (width 0.153) (layer "F.Cu") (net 10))
 (via (at 139.05 150.9308) (size 0.8) (drill 0.4) (layers "F.Cu" "B.Cu") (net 10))
 (segment (start 139.05 150.8997) (end 139.05 150.9308) (width 0.153) (layer "B.Cu") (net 10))
 (segment (start 139.05 150.8997) (end 137.7197 150.8997) (width 0.153) (layer "B.Cu") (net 10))
 (segment (start 147.32 142.75) (end 147.32 146.2018) (width 0.153) (layer "B.Cu") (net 10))
 (segment (start 147.32 146.2018) (end 142.6221 150.8997) (width 0.153) (layer "B.Cu") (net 10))
 (segment (start 137.7197 150.8997) (end 134.62 147.8) (width 0.153) (layer "B.Cu") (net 10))
 (segment (start 142.6221 150.8997) (end 139.05 150.8997) (width 0.153) (layer "B.Cu") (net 10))
 (segment (start 139.375 144.5149) (end 139.375 144.19) (width 0.153) (layer "F.Cu") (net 16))
 (segment (start 138.9944 144.8955) (end 139.375 144.5149) (width 0.153) (layer "F.Cu") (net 16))
 (segment (start 138.4521 144.8955) (end 138.9944 144.8955) (width 0.153) (layer "F.Cu") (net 16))
 (segment (start 137.9235 144.3669) (end 138.4521 144.8955) (width 0.153) (layer "F.Cu") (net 16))
 (segment (start 137.9235 144.2271) (end 137.9235 144.3669) (width 0.153) (layer "F.Cu") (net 16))
 (via (at 137.9235 144.2271) (size 0.8) (drill 0.4) (layers "F.Cu" "B.Cu") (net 16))
 (segment (start 135.4264 141.73) (end 137.9235 144.2271) (width 0.153) (layer "B.Cu") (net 16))
 (segment (start 132.08 141.73) (end 135.4264 141.73) (width 0.153) (layer "B.Cu") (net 16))
 (segment (start 140.025 144.19) (end 140.025 144.4714) (width 0.153) (layer "F.Cu") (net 17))
 (segment (start 140.025 144.4714) (end 140.4937 144.9401) (width 0.153) (layer "F.Cu") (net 17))
 (segment (start 141.4787 144.9401) (end 141.8673 144.5515) (width 0.153) (layer "F.Cu") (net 17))
 (segment (start 140.4937 144.9401) (end 141.4787 144.9401) (width 0.153) (layer "F.Cu") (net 17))
 (via (at 141.8673 144.5515) (size 0.8) (drill 0.4) (layers "F.Cu" "B.Cu") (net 17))
 (segment (start 144.4985 144.5515) (end 141.8673 144.5515) (width 0.153) (layer "B.Cu") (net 17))
 (segment (start 147.32 141.73) (end 144.4985 144.5515) (width 0.153) (layer "B.Cu") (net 17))
 (segment (start 139.7268 150.1929) (end 139.7 150.1661) (width 0.153) (layer "F.Cu") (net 11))
 (segment (start 139.7 152.6786) (end 139.7 151.7018) (width 0.153) (layer "F.Cu") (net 11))
 (segment (start 139.7 151.7018) (end 139.7268 151.675) (width 0.153) (layer "F.Cu") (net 11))
 (segment (start 139.7268 151.675) (end 139.7268 150.1929) (width 0.153) (layer "F.Cu") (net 11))
 (via (at 139.7 150.1661) (size 0.8) (drill 0.4) (layers "F.Cu" "B.Cu") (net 11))
 (segment (start 138.4176 150.1661) (end 139.7 150.1661) (width 0.153) (layer "B.Cu") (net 11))
 (segment (start 136.9915 147.6615) (end 136.9915 148.74) (width 0.153) (layer "B.Cu") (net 11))
 (segment (start 136.9915 148.74) (end 138.4176 150.1661) (width 0.153) (layer "B.Cu") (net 11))
 (segment (start 139.7 150.1661) (end 142.4139 150.1661) (width 0.153) (layer "B.Cu") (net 11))
 (segment (start 142.4139 150.1661) (end 144.78 147.8) (width 0.153) (layer "B.Cu") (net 11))
 (segment (start 132.08 142.75) (end 136.9915 147.6615) (width 0.153) (layer "B.Cu") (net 11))
 (segment (start 141.25 129.04) (end 141.25 130.1309) (width 0.153) (layer "F.Cu") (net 3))
 (segment (start 138.75 130.0175) (end 138.5685 130.199) (width 0.153) (layer "F.Cu") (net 3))
 (segment (start 141.25 130.1309) (end 141.3243 130.2052) (width 0.153) (layer "F.Cu") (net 3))
 (segment (start 141.65 142.565) (end 141.9321 142.565) (width 0.153) (layer "F.Cu") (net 3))
 (segment (start 138.75 129.04) (end 138.75 130.0175) (width 0.153) (layer "F.Cu") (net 3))
 (segment (start 142.3981 142.099) (end 142.3981 135.6241) (width 0.153) (layer "F.Cu") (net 3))
 (segment (start 141.9321 142.565) (end 142.3981 142.099) (width 0.153) (layer "F.Cu") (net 3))
 (via (at 142.3981 135.6241) (size 0.8) (drill 0.4) (layers "F.Cu" "B.Cu") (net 3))
 (via (at 138.5685 130.199) (size 0.8) (drill 0.4) (layers "F.Cu" "B.Cu") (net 3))
 (via (at 141.3243 130.2052) (size 0.8) (drill 0.4) (layers "F.Cu" "B.Cu") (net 3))
 (segment (start 138.5685 132.513) (end 139.528 133.4725) (width 0.153) (layer "B.Cu") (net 3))
 (segment (start 138.75 129.04) (end 138.75 129.8168) (width 0.153) (layer "B.Cu") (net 3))
 (segment (start 138.75 130.0175) (end 138.5685 130.199) (width 0.153) (layer "B.Cu") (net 3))
 (segment (start 138.5685 130.199) (end 138.5685 132.513) (width 0.153) (layer "B.Cu") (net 3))
 (segment (start 141.25 129.04) (end 141.25 129.8168) (width 0.153) (layer "B.Cu") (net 3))
 (segment (start 140.1847 133.4107) (end 141.25 132.3454) (width 0.153) (layer "B.Cu") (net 3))
 (segment (start 141.25 130.2052) (end 141.3243 130.2052) (width 0.153) (layer "B.Cu") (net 3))
 (segment (start 141.25 132.3454) (end 141.25 130.2052) (width 0.153) (layer "B.Cu") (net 3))
 (segment (start 140.1847 133.4107) (end 142.3981 135.6241) (width 0.153) (layer "B.Cu") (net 3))
 (segment (start 138.75 129.8168) (end 138.75 130.0175) (width 0.153) (layer "B.Cu") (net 3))
 (segment (start 140.1229 133.4725) (end 140.1847 133.4107) (width 0.153) (layer "B.Cu") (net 3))
 (segment (start 139.528 133.4725) (end 140.1229 133.4725) (width 0.153) (layer "B.Cu") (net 3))
 (segment (start 141.25 129.8168) (end 141.25 130.2052) (width 0.153) (layer "B.Cu") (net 3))
 (segment (start 137.0442 133.5226) (end 137.0442 141.5399) (width 0.153) (layer "F.Cu") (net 6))
 (segment (start 137.0442 141.5399) (end 137.4193 141.915) (width 0.153) (layer "F.Cu") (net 6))
 (segment (start 137.4193 141.915) (end 137.75 141.915) (width 0.153) (layer "F.Cu") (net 6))
 (segment (start 140.75 129.04) (end 140.75 129.8168) (width 0.153) (layer "F.Cu") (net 6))
 (segment (start 140.75 129.8168) (end 137.0442 133.5226) (width 0.153) (layer "F.Cu") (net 6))
 (segment (start 139.375 140.29) (end 139.375 133.2632) (width 0.153) (layer "F.Cu") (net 8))
 (segment (start 139.375 133.2632) (end 139.8425 132.7957) (width 0.153) (layer "F.Cu") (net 8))
 (via (at 139.8425 132.7957) (size 0.8) (drill 0.4) (layers "F.Cu" "B.Cu") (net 8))
 (segment (start 139.25 129.8168) (end 139.8425 130.4093) (width 0.153) (layer "B.Cu") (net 8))
 (segment (start 139.25 129.04) (end 139.25 129.8168) (width 0.153) (layer "B.Cu") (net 8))
 (segment (start 139.8425 130.4093) (end 139.8425 132.7957) (width 0.153) (layer "B.Cu") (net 8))
 (segment (start 138.3082 151.61) (end 138.4 151.7018) (width 0.153) (layer "F.Cu") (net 9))
 (segment (start 138.3082 149.8791) (end 138.3082 151.61) (width 0.153) (layer "F.Cu") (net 9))
 (segment (start 138.4 152.6786) (end 138.4 151.7018) (width 0.153) (layer "F.Cu") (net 9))
 (segment (start 138.698 149.4893) (end 138.3082 149.8791) (width 0.153) (layer "F.Cu") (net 9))
 (via (at 138.698 149.4893) (size 0.8) (drill 0.4) (layers "F.Cu" "B.Cu") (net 9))
 (segment (start 138.698 149.2409) (end 138.698 149.4893) (width 0.153) (layer "B.Cu") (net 9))
 (segment (start 138.1411 148.684) (end 138.698 149.2409) (width 0.153) (layer "B.Cu") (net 9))
 (segment (start 141.65 140.5112) (end 141.65 141.265) (width 0.153) (layer "F.Cu") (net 19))
 (via (at 141.65 140.5112) (size 0.8) (drill 0.4) (layers "F.Cu" "B.Cu") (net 19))
 (segment (start 140.3047 147.664) (end 140.3047 141.8565) (width 0.153) (layer "B.Cu") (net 19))
 (segment (start 140.3047 141.8565) (end 141.65 140.5112) (width 0.153) (layer "B.Cu") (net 19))
 (segment (start 138.1411 147.664) (end 140.3047 147.664) (width 0.153) (layer "B.Cu") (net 19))
 (segment (start 140.3047 147.664) (end 141.2282 148.5875) (width 0.153) (layer "B.Cu") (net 19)))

